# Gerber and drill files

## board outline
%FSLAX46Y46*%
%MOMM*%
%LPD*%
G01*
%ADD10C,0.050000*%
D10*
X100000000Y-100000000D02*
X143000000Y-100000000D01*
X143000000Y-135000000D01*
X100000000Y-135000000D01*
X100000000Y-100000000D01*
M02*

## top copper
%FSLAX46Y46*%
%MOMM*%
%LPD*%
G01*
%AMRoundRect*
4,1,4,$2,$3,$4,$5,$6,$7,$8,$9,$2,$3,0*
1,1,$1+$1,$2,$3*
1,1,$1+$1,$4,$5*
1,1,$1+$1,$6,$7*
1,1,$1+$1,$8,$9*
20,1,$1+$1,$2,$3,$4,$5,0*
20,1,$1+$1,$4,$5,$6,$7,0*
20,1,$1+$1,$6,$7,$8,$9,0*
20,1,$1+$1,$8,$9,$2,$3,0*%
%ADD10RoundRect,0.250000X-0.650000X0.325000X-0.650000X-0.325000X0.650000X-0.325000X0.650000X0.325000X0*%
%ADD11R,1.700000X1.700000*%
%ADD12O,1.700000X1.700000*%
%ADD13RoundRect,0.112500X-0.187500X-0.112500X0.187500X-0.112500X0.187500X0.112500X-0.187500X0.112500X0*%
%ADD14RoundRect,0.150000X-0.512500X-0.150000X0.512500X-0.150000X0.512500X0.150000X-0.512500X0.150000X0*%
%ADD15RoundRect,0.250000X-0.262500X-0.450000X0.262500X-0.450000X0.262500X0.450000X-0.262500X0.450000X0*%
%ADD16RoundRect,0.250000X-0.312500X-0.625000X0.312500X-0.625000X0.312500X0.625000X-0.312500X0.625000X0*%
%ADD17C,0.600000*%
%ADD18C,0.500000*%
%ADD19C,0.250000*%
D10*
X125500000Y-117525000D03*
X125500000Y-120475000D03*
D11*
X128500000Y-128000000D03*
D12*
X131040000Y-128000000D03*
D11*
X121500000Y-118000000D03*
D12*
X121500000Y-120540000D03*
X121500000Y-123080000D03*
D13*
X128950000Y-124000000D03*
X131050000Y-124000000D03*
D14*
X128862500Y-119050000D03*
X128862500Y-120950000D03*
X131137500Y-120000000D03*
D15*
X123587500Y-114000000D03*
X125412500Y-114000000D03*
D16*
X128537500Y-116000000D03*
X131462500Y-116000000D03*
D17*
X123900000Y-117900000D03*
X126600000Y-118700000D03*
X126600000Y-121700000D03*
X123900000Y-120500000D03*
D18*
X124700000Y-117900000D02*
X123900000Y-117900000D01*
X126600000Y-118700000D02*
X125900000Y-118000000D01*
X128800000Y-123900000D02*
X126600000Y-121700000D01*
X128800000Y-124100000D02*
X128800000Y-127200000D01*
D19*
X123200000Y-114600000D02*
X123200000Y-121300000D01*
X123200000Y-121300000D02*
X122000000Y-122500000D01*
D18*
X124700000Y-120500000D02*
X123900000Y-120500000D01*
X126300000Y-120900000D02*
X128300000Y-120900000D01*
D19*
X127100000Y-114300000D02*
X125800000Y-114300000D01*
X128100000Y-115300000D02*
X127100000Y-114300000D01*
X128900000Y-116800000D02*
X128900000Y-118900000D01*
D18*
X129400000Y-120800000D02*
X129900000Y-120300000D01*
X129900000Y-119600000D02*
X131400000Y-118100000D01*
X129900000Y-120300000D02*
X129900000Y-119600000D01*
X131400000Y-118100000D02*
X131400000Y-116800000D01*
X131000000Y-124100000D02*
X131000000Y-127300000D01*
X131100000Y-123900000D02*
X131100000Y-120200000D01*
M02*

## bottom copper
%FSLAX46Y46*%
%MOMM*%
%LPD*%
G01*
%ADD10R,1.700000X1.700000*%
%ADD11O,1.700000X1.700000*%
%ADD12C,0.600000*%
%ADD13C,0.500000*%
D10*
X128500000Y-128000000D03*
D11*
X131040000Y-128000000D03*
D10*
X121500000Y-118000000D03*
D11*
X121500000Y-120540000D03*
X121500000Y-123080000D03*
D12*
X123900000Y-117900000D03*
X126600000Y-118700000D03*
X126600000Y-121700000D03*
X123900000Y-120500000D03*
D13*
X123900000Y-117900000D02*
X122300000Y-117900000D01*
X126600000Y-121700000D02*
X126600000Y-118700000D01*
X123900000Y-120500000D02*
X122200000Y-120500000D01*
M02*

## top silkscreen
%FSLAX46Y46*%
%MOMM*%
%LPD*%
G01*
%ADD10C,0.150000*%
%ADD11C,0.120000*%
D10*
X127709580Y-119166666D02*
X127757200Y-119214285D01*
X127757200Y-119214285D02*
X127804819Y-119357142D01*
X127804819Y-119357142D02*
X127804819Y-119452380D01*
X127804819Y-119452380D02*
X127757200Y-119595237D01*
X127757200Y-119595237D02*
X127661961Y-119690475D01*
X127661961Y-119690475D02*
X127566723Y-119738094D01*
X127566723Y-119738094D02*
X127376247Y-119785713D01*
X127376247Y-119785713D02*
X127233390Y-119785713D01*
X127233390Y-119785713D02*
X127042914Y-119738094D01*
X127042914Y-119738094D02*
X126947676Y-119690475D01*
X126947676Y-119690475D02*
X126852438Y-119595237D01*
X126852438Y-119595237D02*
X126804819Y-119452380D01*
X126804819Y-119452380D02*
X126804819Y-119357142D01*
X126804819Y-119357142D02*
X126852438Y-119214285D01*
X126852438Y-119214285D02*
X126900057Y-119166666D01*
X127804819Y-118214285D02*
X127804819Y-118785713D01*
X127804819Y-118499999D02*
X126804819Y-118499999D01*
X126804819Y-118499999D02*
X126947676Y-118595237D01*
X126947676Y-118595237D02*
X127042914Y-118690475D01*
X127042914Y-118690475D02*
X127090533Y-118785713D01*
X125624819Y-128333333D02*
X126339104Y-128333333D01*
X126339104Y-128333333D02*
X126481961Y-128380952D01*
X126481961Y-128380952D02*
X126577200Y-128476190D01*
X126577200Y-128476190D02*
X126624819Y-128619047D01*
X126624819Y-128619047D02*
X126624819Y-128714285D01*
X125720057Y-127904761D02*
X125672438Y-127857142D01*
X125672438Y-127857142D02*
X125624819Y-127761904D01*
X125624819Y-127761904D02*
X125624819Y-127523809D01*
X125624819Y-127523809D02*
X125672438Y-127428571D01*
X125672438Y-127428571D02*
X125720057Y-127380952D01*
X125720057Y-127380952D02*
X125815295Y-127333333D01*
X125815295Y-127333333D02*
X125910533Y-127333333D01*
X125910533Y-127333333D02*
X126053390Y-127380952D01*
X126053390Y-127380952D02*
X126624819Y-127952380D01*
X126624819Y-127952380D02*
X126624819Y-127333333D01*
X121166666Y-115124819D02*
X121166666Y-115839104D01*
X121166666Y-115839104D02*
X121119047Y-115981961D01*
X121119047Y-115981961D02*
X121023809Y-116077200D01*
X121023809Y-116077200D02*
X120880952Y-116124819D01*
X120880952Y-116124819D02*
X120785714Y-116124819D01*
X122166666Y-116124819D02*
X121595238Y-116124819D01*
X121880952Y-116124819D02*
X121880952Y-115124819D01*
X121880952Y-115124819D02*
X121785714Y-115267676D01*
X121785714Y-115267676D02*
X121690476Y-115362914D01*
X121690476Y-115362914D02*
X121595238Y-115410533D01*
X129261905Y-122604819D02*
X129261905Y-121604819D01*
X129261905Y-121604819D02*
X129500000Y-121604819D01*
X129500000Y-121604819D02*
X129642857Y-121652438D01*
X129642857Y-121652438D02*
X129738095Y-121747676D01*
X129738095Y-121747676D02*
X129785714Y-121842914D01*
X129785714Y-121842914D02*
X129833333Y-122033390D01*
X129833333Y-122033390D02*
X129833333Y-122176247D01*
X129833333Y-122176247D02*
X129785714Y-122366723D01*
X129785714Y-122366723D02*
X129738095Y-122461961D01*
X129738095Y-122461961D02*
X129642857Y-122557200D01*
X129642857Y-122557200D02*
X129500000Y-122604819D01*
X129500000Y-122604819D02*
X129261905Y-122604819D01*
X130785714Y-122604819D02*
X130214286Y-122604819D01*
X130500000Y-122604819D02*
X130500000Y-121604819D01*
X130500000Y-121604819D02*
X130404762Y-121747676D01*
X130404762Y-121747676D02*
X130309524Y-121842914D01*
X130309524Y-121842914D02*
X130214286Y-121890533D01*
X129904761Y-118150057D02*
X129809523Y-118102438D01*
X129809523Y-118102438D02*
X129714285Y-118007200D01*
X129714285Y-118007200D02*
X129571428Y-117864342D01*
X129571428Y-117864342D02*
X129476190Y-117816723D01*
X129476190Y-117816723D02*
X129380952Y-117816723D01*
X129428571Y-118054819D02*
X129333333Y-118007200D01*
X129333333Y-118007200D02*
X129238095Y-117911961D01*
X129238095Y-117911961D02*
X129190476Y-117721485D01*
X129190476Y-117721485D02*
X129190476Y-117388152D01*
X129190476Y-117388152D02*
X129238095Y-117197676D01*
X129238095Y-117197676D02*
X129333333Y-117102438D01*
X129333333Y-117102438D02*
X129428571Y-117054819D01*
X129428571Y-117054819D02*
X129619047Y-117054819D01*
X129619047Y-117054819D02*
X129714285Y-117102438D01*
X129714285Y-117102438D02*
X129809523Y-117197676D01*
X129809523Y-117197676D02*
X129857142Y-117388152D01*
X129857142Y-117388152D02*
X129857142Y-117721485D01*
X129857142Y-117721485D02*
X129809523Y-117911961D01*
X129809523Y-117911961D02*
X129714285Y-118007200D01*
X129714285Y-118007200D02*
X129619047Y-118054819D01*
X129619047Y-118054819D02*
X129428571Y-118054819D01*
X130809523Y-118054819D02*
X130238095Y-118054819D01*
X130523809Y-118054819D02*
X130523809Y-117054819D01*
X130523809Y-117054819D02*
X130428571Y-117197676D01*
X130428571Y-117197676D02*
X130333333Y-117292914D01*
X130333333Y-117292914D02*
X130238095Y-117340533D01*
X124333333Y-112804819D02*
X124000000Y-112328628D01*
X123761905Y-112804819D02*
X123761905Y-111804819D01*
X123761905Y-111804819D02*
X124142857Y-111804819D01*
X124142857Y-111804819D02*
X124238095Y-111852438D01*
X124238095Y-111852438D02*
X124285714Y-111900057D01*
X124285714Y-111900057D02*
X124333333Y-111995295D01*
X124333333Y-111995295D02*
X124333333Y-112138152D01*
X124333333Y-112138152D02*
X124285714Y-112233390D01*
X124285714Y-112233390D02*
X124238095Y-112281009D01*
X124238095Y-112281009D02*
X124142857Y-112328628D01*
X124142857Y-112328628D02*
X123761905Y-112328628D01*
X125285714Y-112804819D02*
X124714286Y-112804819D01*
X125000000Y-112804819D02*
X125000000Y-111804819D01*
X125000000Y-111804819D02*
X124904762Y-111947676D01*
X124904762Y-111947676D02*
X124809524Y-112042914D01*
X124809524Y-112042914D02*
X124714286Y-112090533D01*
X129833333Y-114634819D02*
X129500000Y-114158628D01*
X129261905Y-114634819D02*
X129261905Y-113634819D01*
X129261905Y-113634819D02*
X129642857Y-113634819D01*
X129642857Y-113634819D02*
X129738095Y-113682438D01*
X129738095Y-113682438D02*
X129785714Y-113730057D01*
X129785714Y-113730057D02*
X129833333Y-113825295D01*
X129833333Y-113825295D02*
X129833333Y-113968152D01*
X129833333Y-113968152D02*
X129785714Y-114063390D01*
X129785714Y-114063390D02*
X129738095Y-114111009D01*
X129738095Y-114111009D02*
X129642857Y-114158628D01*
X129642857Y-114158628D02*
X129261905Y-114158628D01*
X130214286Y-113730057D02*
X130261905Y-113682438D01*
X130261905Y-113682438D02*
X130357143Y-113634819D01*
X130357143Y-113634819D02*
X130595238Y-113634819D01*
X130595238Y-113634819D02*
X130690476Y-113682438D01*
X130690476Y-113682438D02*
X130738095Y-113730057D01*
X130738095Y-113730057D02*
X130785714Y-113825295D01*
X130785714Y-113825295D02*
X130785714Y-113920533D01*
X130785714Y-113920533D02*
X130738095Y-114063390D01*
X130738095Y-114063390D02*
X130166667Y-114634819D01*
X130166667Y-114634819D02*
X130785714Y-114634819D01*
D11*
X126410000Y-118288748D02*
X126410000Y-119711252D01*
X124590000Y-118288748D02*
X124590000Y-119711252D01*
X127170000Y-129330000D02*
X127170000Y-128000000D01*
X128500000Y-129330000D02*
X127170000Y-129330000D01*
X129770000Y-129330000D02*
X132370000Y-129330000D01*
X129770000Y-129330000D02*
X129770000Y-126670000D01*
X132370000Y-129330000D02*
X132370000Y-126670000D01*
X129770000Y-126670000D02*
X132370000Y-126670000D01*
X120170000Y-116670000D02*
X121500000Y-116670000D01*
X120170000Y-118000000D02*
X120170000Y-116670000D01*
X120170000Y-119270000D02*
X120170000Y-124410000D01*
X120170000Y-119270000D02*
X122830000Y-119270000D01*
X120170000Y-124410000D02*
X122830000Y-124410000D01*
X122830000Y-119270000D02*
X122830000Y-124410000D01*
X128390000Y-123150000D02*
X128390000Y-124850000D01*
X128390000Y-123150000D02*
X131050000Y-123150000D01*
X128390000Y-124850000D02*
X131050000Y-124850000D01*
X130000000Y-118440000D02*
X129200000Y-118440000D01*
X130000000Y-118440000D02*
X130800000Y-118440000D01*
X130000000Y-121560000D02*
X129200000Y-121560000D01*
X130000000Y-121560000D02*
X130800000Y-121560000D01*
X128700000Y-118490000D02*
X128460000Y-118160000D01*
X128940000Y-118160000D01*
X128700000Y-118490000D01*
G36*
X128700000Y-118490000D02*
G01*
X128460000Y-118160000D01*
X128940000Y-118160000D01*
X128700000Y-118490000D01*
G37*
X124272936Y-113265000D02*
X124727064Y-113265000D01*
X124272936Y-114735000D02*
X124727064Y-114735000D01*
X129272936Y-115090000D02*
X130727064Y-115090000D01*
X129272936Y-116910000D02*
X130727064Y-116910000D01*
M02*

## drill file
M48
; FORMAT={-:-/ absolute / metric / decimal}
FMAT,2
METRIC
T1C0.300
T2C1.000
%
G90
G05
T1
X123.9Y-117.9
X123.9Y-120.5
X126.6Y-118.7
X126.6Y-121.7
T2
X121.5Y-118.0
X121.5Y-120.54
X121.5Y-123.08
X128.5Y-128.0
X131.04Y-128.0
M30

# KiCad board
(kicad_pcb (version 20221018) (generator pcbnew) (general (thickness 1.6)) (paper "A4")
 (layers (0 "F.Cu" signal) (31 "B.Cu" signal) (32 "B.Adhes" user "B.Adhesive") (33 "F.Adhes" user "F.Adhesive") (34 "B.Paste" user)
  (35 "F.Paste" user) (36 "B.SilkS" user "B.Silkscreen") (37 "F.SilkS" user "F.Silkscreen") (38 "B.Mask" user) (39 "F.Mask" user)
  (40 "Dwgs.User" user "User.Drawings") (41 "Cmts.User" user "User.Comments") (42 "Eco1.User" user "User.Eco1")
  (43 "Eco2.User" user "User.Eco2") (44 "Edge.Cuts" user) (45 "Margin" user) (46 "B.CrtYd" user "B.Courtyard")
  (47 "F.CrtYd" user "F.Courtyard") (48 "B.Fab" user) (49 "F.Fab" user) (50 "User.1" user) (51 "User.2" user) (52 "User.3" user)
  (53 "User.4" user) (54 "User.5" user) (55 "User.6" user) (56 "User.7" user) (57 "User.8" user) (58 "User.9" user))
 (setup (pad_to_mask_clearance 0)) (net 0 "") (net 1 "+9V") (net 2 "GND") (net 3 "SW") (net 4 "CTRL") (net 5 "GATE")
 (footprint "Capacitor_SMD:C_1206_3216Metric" (layer "F.Cu") (at 125.5 119 -90)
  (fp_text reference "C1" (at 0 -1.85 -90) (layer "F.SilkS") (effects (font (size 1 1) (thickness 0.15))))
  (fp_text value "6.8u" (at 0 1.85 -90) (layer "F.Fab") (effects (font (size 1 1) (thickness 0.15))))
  (fp_line (start -0.711252 -0.91) (end 0.711252 -0.91) (stroke (width 0.12) (type solid)) (layer "F.SilkS"))
  (fp_line (start -0.711252 0.91) (end 0.711252 0.91) (stroke (width 0.12) (type solid)) (layer "F.SilkS"))
  (pad "1" smd roundrect (at -1.475 0 270) (size 1.15 1.8) (layers "F.Cu" "F.Paste" "F.Mask") (roundrect_rratio 0.217391) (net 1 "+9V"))
  (pad "2" smd roundrect (at 1.475 0 270) (size 1.15 1.8) (layers "F.Cu" "F.Paste" "F.Mask") (roundrect_rratio 0.217391) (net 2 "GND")))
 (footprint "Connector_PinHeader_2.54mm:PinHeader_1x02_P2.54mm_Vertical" (layer "F.Cu") (at 128.5 128 90)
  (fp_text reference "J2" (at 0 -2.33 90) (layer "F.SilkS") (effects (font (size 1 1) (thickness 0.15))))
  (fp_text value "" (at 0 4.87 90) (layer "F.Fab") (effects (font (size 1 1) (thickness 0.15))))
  (fp_line (start -1.33 -1.33) (end 0 -1.33) (stroke (width 0.12) (type solid)) (layer "F.SilkS"))
  (fp_line (start -1.33 0) (end -1.33 -1.33) (stroke (width 0.12) (type solid)) (layer "F.SilkS"))
  (fp_line (start -1.33 1.27) (end -1.33 3.87) (stroke (width 0.12) (type solid)) (layer "F.SilkS"))
  (fp_line (start -1.33 1.27) (end 1.33 1.27) (stroke (width 0.12) (type solid)) (layer "F.SilkS"))
  (fp_line (start -1.33 3.87) (end 1.33 3.87) (stroke (width 0.12) (type solid)) (layer "F.SilkS"))
  (fp_line (start 1.33 1.27) (end 1.33 3.87) (stroke (width 0.12) (type solid)) (layer "F.SilkS"))
  (pad "1" thru_hole rect (at 0 0 90) (size 1.7 1.7) (drill 1) (layers "*.Cu" "*.Mask") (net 1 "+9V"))
  (pad "2" thru_hole oval (at 0 2.54 90) (size 1.7 1.7) (drill 1) (layers "*.Cu" "*.Mask") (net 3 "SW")))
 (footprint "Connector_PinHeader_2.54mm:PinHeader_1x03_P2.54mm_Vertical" (layer "F.Cu") (at 121.5 118)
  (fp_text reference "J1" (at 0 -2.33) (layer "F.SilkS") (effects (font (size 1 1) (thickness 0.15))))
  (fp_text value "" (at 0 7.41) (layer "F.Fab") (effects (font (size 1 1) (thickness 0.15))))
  (fp_line (start -1.33 -1.33) (end 0 -1.33) (stroke (width 0.12) (type solid)) (layer "F.SilkS"))
  (fp_line (start -1.33 0) (end -1.33 -1.33) (stroke (width 0.12) (type solid)) (layer "F.SilkS"))
  (fp_line (start -1.33 1.27) (end -1.33 6.41) (stroke (width 0.12) (type solid)) (layer "F.SilkS"))
  (fp_line (start -1.33 1.27) (end 1.33 1.27) (stroke (width 0.12) (type solid)) (layer "F.SilkS"))
  (fp_line (start -1.33 6.41) (end 1.33 6.41) (stroke (width 0.12) (type solid)) (layer "F.SilkS"))
  (fp_line (start 1.33 1.27) (end 1.33 6.41) (stroke (width 0.12) (type solid)) (layer "F.SilkS"))
  (pad "1" thru_hole rect (at 0 0) (size 1.7 1.7) (drill 1) (layers "*.Cu" "*.Mask") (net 1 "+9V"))
  (pad "2" thru_hole oval (at 0 2.54) (size 1.7 1.7) (drill 1) (layers "*.Cu" "*.Mask") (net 2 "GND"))
  (pad "3" thru_hole oval (at 0 5.08) (size 1.7 1.7) (drill 1) (layers "*.Cu" "*.Mask") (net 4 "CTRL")))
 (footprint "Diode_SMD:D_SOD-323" (layer "F.Cu") (at 130 124)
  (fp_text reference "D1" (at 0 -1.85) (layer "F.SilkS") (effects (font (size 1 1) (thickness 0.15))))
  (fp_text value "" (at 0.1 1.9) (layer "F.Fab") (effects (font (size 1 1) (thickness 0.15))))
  (fp_line (start -1.61 -0.85) (end -1.61 0.85) (stroke (width 0.12) (type solid)) (layer "F.SilkS"))
  (fp_line (start -1.61 -0.85) (end 1.05 -0.85) (stroke (width 0.12) (type solid)) (layer "F.SilkS"))
  (fp_line (start -1.61 0.85) (end 1.05 0.85) (stroke (width 0.12) (type solid)) (layer "F.SilkS"))
  (pad "1" smd roundrect (at -1.05 0) (size 0.6 0.45) (layers "F.Cu" "F.Paste" "F.Mask") (roundrect_rratio 0.25) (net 1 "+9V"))
  (pad "2" smd roundrect (at 1.05 0) (size 0.6 0.45) (layers "F.Cu" "F.Paste" "F.Mask") (roundrect_rratio 0.25) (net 3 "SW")))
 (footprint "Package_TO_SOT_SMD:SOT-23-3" (layer "F.Cu") (at 130 120)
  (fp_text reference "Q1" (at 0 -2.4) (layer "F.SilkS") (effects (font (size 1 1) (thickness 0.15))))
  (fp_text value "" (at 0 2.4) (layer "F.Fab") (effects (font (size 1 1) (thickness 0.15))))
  (fp_line (start 0 -1.56) (end -0.8 -1.56) (stroke (width 0.12) (type solid)) (layer "F.SilkS"))
  (fp_line (start 0 -1.56) (end 0.8 -1.56) (stroke (width 0.12) (type solid)) (layer "F.SilkS"))
  (fp_line (start 0 1.56) (end -0.8 1.56) (stroke (width 0.12) (type solid)) (layer "F.SilkS"))
  (fp_line (start 0 1.56) (end 0.8 1.56) (stroke (width 0.12) (type solid)) (layer "F.SilkS"))
  (fp_poly
   (pts (xy -1.3 -1.51) (xy -1.54 -1.84) (xy -1.06 -1.84) (xy -1.3 -1.51)) (stroke (width 0.12) (type solid)) (fill solid) (layer "F.SilkS"))
  (pad "1" smd roundrect (at -1.1375 -0.95) (size 1.325 0.6) (layers "F.Cu" "F.Paste" "F.Mask") (roundrect_rratio 0.25) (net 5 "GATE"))
  (pad "2" smd roundrect (at -1.1375 0.95) (size 1.325 0.6) (layers "F.Cu" "F.Paste" "F.Mask") (roundrect_rratio 0.25) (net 2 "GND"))
  (pad "3" smd roundrect (at 1.1375 0) (size 1.325 0.6) (layers "F.Cu" "F.Paste" "F.Mask") (roundrect_rratio 0.25) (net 3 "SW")))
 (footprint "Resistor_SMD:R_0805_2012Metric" (layer "F.Cu") (at 124.5 114)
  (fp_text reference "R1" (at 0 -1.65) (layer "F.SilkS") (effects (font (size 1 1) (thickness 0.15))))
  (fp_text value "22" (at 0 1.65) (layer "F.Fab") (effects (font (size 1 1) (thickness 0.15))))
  (fp_line (start -0.227064 -0.735) (end 0.227064 -0.735) (stroke (width 0.12) (type solid)) (layer "F.SilkS"))
  (fp_line (start -0.227064 0.735) (end 0.227064 0.735) (stroke (width 0.12) (type solid)) (layer "F.SilkS"))
  (pad "1" smd roundrect (at -0.9125 0) (size 1.025 1.4) (layers "F.Cu" "F.Paste" "F.Mask") (roundrect_rratio 0.243902) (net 4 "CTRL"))
  (pad "2" smd roundrect (at 0.9125 0) (size 1.025 1.4) (layers "F.Cu" "F.Paste" "F.Mask") (roundrect_rratio 0.243902) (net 5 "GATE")))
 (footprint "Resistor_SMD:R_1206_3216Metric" (layer "F.Cu") (at 130 116)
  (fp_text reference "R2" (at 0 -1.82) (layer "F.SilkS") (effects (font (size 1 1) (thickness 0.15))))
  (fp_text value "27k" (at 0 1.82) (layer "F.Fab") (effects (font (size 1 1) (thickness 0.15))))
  (fp_line (start -0.727064 -0.91) (end 0.727064 -0.91) (stroke (width 0.12) (type solid)) (layer "F.SilkS"))
  (fp_line (start -0.727064 0.91) (end 0.727064 0.91) (stroke (width 0.12) (type solid)) (layer "F.SilkS"))
  (pad "1" smd roundrect (at -1.4625 0) (size 1.125 1.75) (layers "F.Cu" "F.Paste" "F.Mask") (roundrect_rratio 0.222222) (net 5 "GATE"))
  (pad "2" smd roundrect (at 1.4625 0) (size 1.125 1.75) (layers "F.Cu" "F.Paste" "F.Mask") (roundrect_rratio 0.222222) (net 2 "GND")))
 (gr_rect (start 100 100) (end 143 135) (stroke (width 0.05) (type default)) (fill none) (layer "Edge.Cuts"))
 (segment (start 124.7 117.9) (end 123.9 117.9) (width 0.5) (layer "F.Cu") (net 1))
 (segment (start 126.6 118.7) (end 125.9 118) (width 0.5) (layer "F.Cu") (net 1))
 (segment (start 128.8 123.9) (end 126.6 121.7) (width 0.5) (layer "F.Cu") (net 1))
 (segment (start 128.8 124.1) (end 128.8 127.2) (width 0.5) (layer "F.Cu") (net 1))
 (via (at 123.9 117.9) (size 0.6) (drill 0.3) (layers "F.Cu" "B.Cu") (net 1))
 (via (at 126.6 118.7) (size 0.6) (drill 0.3) (layers "F.Cu" "B.Cu") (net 1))
 (via (at 126.6 121.7) (size 0.6) (drill 0.3) (layers "F.Cu" "B.Cu") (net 1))
 (segment (start 123.2 114.6) (end 123.2 121.3) (width 0.25) (layer "F.Cu") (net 4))
 (segment (start 123.2 121.3) (end 122 122.5) (width 0.25) (layer "F.Cu") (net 4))
 (segment (start 123.9 117.9) (end 122.3 117.9) (width 0.5) (layer "B.Cu") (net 1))
 (segment (start 124.7 120.5) (end 123.9 120.5) (width 0.5) (layer "F.Cu") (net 2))
 (segment (start 126.3 120.9) (end 128.3 120.9) (width 0.5) (layer "F.Cu") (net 2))
 (segment (start 126.6 121.7) (end 126.6 118.7) (width 0.5) (layer "B.Cu") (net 1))
 (segment (start 127.1 114.3) (end 125.8 114.3) (width 0.25) (layer "F.Cu") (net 5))
 (segment (start 128.1 115.3) (end 127.1 114.3) (width 0.25) (layer "F.Cu") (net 5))
 (segment (start 128.9 116.8) (end 128.9 118.9) (width 0.25) (layer "F.Cu") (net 5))
 (segment (start 129.4 120.8) (end 129.9 120.3) (width 0.5) (layer "F.Cu") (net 2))
 (segment (start 129.9 119.6) (end 131.4 118.1) (width 0.5) (layer "F.Cu") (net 2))
 (segment (start 129.9 120.3) (end 129.9 119.6) (width 0.5) (layer "F.Cu") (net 2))
 (segment (start 131.4 118.1) (end 131.4 116.8) (width 0.5) (layer "F.Cu") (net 2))
 (via (at 123.9 120.5) (size 0.6) (drill 0.3) (layers "F.Cu" "B.Cu") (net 2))
 (segment (start 123.9 120.5) (end 122.2 120.5) (width 0.5) (layer "B.Cu") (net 2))
 (segment (start 131 124.1) (end 131 127.3) (width 0.5) (layer "F.Cu") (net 3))
 (segment (start 131.1 123.9) (end 131.1 120.2) (width 0.5) (layer "F.Cu") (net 3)))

